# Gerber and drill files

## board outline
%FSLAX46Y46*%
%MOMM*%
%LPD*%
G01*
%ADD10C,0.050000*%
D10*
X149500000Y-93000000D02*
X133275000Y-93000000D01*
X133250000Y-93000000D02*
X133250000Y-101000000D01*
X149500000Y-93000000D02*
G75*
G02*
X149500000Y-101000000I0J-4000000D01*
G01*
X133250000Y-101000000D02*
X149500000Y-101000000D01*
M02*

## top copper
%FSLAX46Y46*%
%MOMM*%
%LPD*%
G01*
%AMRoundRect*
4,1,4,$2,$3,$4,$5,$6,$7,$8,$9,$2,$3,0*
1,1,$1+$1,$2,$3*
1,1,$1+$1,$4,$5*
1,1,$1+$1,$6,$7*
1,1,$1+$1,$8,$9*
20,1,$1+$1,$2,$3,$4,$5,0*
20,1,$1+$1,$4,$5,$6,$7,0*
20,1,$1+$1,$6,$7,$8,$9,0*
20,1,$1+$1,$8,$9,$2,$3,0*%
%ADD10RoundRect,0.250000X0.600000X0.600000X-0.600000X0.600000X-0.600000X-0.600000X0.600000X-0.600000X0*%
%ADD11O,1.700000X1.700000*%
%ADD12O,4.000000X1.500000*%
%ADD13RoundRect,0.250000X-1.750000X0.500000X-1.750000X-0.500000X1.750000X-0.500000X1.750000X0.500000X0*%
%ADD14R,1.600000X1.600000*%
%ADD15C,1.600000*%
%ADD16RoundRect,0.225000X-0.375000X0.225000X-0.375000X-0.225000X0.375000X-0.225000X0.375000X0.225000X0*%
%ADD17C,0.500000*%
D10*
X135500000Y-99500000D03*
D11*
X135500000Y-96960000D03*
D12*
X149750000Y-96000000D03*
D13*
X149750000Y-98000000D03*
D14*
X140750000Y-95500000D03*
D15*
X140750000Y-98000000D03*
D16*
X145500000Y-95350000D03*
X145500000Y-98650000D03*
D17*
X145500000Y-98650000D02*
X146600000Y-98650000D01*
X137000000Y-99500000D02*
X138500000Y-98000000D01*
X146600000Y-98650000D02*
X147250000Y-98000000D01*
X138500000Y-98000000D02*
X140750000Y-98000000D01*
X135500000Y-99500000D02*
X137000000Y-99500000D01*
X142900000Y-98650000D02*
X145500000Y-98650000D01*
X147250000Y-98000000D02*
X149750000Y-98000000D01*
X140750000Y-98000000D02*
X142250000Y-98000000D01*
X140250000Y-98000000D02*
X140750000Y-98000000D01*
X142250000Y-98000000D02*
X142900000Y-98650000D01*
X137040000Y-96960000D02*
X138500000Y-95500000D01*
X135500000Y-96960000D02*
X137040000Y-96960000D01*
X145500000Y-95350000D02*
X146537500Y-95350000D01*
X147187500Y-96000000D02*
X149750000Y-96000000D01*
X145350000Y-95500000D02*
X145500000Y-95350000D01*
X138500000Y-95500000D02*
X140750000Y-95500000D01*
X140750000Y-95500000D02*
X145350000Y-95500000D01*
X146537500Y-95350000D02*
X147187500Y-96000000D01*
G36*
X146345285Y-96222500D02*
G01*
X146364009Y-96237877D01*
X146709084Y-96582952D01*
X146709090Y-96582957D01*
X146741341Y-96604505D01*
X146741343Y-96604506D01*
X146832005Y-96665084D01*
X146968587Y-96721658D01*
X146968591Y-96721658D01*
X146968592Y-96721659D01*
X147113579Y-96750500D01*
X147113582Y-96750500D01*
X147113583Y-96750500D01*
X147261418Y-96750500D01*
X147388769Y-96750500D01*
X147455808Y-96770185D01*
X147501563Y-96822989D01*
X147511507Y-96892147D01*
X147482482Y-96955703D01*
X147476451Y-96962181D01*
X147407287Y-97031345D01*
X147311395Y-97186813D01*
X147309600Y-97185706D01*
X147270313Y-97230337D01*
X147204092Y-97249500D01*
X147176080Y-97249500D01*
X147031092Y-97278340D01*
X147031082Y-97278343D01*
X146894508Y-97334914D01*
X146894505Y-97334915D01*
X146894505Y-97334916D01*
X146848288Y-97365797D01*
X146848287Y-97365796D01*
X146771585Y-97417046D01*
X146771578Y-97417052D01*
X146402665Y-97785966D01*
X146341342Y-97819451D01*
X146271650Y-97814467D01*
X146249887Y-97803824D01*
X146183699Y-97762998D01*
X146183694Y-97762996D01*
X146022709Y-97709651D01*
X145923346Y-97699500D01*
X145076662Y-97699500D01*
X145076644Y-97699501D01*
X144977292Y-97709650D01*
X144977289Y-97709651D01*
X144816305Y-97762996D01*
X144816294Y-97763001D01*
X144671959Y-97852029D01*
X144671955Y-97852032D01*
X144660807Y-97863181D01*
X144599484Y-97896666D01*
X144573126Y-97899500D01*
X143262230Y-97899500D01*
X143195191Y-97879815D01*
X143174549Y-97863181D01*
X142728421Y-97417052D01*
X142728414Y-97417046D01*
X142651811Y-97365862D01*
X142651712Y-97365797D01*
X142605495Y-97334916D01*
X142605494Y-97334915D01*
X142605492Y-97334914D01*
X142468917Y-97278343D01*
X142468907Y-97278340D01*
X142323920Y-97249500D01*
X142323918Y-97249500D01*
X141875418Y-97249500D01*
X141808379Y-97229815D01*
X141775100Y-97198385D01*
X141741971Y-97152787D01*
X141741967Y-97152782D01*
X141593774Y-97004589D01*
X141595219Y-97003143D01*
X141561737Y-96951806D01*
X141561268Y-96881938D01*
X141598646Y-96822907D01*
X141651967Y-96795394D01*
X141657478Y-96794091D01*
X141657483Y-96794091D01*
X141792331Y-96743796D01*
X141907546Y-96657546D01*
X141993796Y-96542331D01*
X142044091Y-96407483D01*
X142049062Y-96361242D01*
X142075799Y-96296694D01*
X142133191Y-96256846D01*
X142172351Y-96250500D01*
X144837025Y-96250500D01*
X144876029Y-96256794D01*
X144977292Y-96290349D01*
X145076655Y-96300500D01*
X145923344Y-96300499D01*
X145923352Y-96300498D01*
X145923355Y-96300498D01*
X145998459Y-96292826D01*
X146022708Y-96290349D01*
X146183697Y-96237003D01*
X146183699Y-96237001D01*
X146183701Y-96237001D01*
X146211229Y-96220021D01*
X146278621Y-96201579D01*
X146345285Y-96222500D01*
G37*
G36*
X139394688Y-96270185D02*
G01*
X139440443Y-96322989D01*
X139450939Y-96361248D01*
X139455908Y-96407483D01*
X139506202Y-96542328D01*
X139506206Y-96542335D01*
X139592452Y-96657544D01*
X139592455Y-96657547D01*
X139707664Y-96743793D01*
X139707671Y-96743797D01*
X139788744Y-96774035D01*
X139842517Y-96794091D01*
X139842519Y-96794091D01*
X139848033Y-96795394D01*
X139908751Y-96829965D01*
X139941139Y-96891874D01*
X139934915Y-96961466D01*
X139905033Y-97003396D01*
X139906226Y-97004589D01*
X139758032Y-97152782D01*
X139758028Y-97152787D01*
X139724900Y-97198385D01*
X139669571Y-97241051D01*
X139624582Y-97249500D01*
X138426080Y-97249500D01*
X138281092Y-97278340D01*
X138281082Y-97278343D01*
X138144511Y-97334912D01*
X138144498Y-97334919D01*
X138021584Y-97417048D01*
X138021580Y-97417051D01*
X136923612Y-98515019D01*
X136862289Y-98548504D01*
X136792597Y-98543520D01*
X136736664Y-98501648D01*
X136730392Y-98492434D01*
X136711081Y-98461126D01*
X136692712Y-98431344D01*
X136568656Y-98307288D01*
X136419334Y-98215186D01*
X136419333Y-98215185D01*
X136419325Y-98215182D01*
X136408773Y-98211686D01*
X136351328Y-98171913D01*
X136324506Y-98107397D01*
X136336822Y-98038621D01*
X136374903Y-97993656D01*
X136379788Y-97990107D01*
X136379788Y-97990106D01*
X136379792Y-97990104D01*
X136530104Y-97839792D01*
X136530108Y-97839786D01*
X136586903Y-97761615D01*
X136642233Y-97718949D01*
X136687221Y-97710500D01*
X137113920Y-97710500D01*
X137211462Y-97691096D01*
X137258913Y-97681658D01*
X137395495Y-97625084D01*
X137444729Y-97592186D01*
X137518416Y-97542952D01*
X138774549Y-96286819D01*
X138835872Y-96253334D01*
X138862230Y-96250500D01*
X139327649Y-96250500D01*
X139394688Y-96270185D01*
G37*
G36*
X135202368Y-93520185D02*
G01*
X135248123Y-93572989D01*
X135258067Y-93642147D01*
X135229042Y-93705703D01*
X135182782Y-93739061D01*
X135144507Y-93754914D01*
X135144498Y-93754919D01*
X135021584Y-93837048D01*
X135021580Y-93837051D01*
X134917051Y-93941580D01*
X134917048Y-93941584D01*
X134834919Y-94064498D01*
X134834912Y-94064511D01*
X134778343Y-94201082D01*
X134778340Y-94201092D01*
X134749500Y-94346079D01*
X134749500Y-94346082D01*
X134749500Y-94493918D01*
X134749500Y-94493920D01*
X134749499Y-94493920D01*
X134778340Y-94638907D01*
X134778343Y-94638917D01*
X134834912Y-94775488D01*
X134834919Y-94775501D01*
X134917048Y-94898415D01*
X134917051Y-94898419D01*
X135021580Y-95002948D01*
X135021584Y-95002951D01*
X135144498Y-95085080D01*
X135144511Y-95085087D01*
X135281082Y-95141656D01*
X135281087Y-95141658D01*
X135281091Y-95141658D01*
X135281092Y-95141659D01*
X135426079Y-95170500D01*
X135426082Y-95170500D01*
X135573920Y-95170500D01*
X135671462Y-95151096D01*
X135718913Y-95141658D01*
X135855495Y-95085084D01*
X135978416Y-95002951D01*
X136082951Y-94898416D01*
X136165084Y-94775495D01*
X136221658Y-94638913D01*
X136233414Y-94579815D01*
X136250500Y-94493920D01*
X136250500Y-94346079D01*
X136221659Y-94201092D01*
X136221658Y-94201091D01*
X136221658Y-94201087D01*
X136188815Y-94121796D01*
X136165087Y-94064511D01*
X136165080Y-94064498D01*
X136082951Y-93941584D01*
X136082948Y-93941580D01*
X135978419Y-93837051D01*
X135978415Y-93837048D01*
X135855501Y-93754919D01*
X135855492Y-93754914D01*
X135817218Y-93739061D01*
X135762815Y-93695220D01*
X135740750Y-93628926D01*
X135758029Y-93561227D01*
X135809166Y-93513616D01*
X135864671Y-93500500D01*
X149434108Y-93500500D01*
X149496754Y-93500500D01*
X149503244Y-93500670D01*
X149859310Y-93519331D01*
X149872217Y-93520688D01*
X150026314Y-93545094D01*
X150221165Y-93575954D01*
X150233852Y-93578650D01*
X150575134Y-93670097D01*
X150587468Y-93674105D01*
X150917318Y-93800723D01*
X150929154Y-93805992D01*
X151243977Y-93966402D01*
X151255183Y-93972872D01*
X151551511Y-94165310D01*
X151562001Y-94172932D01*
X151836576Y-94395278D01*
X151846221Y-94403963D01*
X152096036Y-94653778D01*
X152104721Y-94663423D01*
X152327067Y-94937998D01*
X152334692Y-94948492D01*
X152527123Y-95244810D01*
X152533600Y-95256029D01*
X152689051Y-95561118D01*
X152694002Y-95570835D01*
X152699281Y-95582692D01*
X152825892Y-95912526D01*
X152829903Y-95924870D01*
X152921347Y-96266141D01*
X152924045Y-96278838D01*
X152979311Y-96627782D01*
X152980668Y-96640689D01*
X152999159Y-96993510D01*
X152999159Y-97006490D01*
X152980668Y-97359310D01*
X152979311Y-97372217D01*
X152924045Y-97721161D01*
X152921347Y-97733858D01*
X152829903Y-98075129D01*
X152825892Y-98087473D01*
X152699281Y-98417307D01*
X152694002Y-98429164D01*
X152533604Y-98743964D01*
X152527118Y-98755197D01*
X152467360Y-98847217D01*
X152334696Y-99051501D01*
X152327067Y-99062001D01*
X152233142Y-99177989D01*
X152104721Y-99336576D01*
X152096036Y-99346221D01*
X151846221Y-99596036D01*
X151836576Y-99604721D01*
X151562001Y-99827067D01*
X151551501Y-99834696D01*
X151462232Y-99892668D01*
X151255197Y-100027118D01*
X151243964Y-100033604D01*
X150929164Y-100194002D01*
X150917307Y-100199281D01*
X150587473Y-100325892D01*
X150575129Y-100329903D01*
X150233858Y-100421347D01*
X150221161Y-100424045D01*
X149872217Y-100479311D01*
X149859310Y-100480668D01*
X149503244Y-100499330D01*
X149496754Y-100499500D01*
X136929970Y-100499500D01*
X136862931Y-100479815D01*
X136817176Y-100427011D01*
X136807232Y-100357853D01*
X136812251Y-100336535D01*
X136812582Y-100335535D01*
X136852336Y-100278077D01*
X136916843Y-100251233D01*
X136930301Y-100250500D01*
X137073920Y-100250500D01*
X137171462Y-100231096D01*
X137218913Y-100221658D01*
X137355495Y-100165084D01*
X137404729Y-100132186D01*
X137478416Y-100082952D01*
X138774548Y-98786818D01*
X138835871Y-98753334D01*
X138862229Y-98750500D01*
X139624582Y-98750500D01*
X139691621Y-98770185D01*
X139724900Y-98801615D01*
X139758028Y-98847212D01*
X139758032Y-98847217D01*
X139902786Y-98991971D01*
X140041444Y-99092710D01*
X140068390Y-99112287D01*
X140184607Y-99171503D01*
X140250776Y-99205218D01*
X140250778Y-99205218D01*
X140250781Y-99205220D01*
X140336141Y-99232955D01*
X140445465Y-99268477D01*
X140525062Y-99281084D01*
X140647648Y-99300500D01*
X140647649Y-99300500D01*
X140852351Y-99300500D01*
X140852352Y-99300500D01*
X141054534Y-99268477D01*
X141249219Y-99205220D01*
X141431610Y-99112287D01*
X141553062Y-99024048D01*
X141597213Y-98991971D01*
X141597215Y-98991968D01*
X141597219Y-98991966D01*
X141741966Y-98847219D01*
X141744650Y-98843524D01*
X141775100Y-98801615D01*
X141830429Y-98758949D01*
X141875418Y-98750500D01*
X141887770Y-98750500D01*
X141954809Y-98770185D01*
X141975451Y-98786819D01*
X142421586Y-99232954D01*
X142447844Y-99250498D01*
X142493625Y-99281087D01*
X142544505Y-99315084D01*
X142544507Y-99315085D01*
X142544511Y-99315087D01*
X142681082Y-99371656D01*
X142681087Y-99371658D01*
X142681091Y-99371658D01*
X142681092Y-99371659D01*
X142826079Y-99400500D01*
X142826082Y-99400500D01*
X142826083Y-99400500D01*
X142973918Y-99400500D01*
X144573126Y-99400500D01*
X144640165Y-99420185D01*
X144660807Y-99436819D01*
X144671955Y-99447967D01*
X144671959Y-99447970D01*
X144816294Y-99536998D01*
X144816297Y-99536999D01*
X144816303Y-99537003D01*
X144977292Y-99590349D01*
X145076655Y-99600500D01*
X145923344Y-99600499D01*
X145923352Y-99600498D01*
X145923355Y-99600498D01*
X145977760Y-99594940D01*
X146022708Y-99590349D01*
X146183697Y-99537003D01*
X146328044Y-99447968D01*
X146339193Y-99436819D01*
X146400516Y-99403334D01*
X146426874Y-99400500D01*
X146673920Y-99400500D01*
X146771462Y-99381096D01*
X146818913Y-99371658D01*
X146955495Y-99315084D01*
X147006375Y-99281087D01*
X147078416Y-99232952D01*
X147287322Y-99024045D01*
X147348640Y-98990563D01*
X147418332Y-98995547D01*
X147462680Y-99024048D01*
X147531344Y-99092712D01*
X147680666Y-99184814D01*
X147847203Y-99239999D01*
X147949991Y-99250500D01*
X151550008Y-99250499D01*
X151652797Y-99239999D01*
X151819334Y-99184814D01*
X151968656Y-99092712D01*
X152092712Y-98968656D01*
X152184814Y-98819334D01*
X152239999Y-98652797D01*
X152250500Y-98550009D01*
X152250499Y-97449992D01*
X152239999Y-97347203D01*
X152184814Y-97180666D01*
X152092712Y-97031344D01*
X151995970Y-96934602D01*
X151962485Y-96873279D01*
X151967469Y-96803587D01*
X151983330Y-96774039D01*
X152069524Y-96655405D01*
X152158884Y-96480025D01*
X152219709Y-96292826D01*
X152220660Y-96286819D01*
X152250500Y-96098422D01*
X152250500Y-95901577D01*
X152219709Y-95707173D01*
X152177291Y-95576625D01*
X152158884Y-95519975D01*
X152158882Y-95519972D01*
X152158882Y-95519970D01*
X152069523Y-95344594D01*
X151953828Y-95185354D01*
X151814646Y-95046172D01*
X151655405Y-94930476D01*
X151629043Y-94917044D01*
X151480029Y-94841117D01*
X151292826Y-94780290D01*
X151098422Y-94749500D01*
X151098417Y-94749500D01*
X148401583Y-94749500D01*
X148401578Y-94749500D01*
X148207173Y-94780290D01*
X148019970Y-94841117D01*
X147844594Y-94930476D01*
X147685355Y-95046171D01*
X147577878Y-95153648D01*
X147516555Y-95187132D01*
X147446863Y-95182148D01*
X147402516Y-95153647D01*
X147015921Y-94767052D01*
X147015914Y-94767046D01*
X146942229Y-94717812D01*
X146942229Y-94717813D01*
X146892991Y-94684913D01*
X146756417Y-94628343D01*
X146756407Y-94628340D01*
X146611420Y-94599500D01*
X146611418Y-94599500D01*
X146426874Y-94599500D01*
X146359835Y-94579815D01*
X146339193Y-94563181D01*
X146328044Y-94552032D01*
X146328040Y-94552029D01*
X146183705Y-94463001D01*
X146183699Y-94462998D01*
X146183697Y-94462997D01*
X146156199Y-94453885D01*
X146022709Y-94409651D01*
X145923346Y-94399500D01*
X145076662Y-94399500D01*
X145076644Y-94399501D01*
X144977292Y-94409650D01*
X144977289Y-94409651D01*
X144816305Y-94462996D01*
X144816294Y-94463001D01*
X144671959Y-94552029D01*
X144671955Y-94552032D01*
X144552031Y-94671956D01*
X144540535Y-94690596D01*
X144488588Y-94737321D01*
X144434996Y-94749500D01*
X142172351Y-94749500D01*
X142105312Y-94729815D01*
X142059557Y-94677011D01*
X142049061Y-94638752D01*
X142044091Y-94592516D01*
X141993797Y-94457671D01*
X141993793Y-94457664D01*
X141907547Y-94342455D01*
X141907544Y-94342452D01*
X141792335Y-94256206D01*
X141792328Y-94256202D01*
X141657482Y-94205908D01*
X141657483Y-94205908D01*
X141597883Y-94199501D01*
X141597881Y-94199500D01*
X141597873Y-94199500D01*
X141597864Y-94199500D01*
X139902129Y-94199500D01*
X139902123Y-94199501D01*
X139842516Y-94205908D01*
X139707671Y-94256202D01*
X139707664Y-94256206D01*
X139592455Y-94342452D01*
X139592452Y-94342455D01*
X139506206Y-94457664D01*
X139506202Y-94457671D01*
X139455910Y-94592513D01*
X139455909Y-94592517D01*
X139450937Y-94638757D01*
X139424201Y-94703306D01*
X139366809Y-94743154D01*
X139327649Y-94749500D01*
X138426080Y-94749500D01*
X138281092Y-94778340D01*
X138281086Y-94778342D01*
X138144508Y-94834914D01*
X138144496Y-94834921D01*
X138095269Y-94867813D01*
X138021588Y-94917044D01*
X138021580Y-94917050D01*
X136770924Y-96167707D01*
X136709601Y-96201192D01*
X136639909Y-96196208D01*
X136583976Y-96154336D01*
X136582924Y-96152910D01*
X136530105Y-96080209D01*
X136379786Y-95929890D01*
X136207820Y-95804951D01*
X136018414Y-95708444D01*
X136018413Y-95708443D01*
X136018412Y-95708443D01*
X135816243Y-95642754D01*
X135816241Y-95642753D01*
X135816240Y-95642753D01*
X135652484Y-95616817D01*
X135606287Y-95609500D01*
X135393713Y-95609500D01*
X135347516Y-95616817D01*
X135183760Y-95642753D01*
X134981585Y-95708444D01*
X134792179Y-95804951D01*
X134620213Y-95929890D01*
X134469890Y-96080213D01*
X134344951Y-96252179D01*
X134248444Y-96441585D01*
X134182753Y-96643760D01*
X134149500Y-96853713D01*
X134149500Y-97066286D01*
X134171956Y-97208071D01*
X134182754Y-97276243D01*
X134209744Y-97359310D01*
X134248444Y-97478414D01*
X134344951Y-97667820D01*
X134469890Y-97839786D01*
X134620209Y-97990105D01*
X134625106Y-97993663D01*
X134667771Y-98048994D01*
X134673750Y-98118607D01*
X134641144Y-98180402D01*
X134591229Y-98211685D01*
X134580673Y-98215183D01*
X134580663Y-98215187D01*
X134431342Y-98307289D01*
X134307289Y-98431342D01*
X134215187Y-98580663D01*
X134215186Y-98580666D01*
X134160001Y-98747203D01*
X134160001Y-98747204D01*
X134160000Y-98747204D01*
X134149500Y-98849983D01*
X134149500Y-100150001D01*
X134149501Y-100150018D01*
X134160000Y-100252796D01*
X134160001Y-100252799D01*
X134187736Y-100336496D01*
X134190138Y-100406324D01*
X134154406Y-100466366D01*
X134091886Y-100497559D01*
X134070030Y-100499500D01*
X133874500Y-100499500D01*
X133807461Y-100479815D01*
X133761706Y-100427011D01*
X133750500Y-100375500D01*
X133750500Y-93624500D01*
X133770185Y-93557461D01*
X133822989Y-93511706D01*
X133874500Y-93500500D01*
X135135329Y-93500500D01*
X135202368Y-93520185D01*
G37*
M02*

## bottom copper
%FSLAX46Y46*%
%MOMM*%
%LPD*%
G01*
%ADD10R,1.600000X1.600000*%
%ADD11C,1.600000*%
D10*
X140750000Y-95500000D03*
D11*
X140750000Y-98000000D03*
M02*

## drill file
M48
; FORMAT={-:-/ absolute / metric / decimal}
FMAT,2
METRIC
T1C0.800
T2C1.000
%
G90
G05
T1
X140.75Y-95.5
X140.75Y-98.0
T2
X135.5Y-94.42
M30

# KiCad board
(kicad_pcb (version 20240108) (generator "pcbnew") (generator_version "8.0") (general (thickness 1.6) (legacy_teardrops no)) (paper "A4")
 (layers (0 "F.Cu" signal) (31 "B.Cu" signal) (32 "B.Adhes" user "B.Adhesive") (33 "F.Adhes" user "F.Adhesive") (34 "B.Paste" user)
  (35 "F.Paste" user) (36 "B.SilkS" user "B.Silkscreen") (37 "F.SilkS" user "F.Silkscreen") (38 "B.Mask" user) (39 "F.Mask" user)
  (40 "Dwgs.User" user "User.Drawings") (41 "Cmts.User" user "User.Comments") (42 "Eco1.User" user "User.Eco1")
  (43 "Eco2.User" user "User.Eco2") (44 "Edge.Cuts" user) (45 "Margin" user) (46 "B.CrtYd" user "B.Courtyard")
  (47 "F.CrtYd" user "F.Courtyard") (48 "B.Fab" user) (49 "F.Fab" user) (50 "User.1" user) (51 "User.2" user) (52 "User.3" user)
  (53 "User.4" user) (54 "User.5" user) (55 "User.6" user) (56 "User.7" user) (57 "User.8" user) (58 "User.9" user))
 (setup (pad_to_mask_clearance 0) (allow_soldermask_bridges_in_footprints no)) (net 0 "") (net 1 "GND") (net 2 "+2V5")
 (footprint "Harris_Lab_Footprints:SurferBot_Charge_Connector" (layer "F.Cu") (at 135.5 99.5 180)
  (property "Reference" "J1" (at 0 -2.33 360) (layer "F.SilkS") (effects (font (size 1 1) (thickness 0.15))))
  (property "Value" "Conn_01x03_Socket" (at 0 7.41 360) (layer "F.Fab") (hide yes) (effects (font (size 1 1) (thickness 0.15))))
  (pad "" np_thru_hole oval (at 0 5.08 180) (size 1.7 1.7) (drill 1) (layers "F.Mask") (zone_connect 0))
  (pad "1" smd roundrect (at 0 0 180) (size 1.7 1.7) (layers "F.Cu" "F.Paste" "F.Mask") (roundrect_rratio 0.1470588235) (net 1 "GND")
   (solder_mask_margin 0.2))
  (pad "2" smd oval (at 0 2.54 180) (size 1.7 1.7) (layers "F.Cu" "F.Paste" "F.Mask") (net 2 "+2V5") (solder_mask_margin 0.2)))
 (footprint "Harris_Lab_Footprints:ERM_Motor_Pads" (layer "F.Cu") (at 149.75 97 -90)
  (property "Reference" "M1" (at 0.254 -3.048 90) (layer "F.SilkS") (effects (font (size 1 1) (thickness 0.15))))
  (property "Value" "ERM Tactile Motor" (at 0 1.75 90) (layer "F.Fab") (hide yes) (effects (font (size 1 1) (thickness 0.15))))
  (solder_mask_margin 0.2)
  (pad "1" smd oval (at -1 0 270) (size 1.5 4) (layers "F.Cu" "F.Mask") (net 2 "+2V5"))
  (pad "2" smd roundrect (at 1 0 270) (size 1.5 4) (layers "F.Cu" "F.Mask") (roundrect_rratio 0.1666666667) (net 1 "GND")))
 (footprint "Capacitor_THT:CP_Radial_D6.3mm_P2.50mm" (layer "F.Cu") (at 140.75 95.5 -90)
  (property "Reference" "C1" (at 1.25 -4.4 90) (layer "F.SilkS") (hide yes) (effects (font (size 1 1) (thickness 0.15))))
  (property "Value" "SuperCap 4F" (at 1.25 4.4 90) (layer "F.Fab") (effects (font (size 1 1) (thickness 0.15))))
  (pad "1" thru_hole rect (at 0 0 270) (size 1.6 1.6) (drill 0.8) (layers "*.Cu" "*.Mask") (remove_unused_layers no) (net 2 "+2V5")
   (solder_mask_margin 0.2))
  (pad "2" thru_hole circle (at 2.5 0 270) (size 1.6 1.6) (drill 0.8) (layers "*.Cu" "*.Mask") (remove_unused_layers no) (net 1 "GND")
   (solder_mask_margin 0.2)))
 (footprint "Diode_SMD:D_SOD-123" (layer "F.Cu") (at 145.5 97 -90)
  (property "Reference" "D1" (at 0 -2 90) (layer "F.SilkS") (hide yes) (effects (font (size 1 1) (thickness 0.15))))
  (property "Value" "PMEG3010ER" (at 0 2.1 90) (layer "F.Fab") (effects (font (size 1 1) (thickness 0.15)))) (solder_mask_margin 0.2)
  (pad "1" smd roundrect (at -1.65 0 270) (size 0.9 1.2) (layers "F.Cu" "F.Paste" "F.Mask") (roundrect_rratio 0.25) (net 2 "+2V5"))
  (pad "2" smd roundrect (at 1.65 0 270) (size 0.9 1.2) (layers "F.Cu" "F.Paste" "F.Mask") (roundrect_rratio 0.25) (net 1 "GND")))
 (gr_line (start 149.5 93) (end 133.275 93) (stroke (width 0.05) (type default)) (layer "Edge.Cuts"))
 (gr_line (start 133.25 93) (end 133.25 101) (stroke (width 0.05) (type default)) (layer "Edge.Cuts"))
 (gr_arc (start 149.5 93) (mid 153.5 97) (end 149.5 101) (stroke (width 0.05) (type default)) (layer "Edge.Cuts"))
 (gr_line (start 133.25 101) (end 149.5 101) (stroke (width 0.05) (type default)) (layer "Edge.Cuts"))
 (segment (start 145.5 98.65) (end 146.6 98.65) (width 0.5) (layer "F.Cu") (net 1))
 (segment (start 137 99.5) (end 138.5 98) (width 0.5) (layer "F.Cu") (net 1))
 (segment (start 146.6 98.65) (end 147.25 98) (width 0.5) (layer "F.Cu") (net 1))
 (segment (start 138.5 98) (end 140.75 98) (width 0.5) (layer "F.Cu") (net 1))
 (segment (start 135.5 99.5) (end 137 99.5) (width 0.5) (layer "F.Cu") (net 1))
 (segment (start 142.9 98.65) (end 145.5 98.65) (width 0.5) (layer "F.Cu") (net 1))
 (segment (start 147.25 98) (end 149.75 98) (width 0.5) (layer "F.Cu") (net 1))
 (segment (start 140.75 98) (end 142.25 98) (width 0.5) (layer "F.Cu") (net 1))
 (segment (start 140.25 98) (end 140.75 98) (width 0.5) (layer "F.Cu") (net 1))
 (segment (start 142.25 98) (end 142.9 98.65) (width 0.5) (layer "F.Cu") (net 1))
 (segment (start 137.04 96.96) (end 138.5 95.5) (width 0.5) (layer "F.Cu") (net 2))
 (segment (start 135.5 96.96) (end 137.04 96.96) (width 0.5) (layer "F.Cu") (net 2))
 (segment (start 145.5 95.35) (end 146.5375 95.35) (width 0.5) (layer "F.Cu") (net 2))
 (segment (start 147.1875 96) (end 149.75 96) (width 0.5) (layer "F.Cu") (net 2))
 (segment (start 145.35 95.5) (end 145.5 95.35) (width 0.5) (layer "F.Cu") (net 2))
 (segment (start 138.5 95.5) (end 140.75 95.5) (width 0.5) (layer "F.Cu") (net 2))
 (segment (start 140.75 95.5) (end 145.35 95.5) (width 0.5) (layer "F.Cu") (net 2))
 (segment (start 146.5375 95.35) (end 147.1875 96) (width 0.5) (layer "F.Cu") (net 2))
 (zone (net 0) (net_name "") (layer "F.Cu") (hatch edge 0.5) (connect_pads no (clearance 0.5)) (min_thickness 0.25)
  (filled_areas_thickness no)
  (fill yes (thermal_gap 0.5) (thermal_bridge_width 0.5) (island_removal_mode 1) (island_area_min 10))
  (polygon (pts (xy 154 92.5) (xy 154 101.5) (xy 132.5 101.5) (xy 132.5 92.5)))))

